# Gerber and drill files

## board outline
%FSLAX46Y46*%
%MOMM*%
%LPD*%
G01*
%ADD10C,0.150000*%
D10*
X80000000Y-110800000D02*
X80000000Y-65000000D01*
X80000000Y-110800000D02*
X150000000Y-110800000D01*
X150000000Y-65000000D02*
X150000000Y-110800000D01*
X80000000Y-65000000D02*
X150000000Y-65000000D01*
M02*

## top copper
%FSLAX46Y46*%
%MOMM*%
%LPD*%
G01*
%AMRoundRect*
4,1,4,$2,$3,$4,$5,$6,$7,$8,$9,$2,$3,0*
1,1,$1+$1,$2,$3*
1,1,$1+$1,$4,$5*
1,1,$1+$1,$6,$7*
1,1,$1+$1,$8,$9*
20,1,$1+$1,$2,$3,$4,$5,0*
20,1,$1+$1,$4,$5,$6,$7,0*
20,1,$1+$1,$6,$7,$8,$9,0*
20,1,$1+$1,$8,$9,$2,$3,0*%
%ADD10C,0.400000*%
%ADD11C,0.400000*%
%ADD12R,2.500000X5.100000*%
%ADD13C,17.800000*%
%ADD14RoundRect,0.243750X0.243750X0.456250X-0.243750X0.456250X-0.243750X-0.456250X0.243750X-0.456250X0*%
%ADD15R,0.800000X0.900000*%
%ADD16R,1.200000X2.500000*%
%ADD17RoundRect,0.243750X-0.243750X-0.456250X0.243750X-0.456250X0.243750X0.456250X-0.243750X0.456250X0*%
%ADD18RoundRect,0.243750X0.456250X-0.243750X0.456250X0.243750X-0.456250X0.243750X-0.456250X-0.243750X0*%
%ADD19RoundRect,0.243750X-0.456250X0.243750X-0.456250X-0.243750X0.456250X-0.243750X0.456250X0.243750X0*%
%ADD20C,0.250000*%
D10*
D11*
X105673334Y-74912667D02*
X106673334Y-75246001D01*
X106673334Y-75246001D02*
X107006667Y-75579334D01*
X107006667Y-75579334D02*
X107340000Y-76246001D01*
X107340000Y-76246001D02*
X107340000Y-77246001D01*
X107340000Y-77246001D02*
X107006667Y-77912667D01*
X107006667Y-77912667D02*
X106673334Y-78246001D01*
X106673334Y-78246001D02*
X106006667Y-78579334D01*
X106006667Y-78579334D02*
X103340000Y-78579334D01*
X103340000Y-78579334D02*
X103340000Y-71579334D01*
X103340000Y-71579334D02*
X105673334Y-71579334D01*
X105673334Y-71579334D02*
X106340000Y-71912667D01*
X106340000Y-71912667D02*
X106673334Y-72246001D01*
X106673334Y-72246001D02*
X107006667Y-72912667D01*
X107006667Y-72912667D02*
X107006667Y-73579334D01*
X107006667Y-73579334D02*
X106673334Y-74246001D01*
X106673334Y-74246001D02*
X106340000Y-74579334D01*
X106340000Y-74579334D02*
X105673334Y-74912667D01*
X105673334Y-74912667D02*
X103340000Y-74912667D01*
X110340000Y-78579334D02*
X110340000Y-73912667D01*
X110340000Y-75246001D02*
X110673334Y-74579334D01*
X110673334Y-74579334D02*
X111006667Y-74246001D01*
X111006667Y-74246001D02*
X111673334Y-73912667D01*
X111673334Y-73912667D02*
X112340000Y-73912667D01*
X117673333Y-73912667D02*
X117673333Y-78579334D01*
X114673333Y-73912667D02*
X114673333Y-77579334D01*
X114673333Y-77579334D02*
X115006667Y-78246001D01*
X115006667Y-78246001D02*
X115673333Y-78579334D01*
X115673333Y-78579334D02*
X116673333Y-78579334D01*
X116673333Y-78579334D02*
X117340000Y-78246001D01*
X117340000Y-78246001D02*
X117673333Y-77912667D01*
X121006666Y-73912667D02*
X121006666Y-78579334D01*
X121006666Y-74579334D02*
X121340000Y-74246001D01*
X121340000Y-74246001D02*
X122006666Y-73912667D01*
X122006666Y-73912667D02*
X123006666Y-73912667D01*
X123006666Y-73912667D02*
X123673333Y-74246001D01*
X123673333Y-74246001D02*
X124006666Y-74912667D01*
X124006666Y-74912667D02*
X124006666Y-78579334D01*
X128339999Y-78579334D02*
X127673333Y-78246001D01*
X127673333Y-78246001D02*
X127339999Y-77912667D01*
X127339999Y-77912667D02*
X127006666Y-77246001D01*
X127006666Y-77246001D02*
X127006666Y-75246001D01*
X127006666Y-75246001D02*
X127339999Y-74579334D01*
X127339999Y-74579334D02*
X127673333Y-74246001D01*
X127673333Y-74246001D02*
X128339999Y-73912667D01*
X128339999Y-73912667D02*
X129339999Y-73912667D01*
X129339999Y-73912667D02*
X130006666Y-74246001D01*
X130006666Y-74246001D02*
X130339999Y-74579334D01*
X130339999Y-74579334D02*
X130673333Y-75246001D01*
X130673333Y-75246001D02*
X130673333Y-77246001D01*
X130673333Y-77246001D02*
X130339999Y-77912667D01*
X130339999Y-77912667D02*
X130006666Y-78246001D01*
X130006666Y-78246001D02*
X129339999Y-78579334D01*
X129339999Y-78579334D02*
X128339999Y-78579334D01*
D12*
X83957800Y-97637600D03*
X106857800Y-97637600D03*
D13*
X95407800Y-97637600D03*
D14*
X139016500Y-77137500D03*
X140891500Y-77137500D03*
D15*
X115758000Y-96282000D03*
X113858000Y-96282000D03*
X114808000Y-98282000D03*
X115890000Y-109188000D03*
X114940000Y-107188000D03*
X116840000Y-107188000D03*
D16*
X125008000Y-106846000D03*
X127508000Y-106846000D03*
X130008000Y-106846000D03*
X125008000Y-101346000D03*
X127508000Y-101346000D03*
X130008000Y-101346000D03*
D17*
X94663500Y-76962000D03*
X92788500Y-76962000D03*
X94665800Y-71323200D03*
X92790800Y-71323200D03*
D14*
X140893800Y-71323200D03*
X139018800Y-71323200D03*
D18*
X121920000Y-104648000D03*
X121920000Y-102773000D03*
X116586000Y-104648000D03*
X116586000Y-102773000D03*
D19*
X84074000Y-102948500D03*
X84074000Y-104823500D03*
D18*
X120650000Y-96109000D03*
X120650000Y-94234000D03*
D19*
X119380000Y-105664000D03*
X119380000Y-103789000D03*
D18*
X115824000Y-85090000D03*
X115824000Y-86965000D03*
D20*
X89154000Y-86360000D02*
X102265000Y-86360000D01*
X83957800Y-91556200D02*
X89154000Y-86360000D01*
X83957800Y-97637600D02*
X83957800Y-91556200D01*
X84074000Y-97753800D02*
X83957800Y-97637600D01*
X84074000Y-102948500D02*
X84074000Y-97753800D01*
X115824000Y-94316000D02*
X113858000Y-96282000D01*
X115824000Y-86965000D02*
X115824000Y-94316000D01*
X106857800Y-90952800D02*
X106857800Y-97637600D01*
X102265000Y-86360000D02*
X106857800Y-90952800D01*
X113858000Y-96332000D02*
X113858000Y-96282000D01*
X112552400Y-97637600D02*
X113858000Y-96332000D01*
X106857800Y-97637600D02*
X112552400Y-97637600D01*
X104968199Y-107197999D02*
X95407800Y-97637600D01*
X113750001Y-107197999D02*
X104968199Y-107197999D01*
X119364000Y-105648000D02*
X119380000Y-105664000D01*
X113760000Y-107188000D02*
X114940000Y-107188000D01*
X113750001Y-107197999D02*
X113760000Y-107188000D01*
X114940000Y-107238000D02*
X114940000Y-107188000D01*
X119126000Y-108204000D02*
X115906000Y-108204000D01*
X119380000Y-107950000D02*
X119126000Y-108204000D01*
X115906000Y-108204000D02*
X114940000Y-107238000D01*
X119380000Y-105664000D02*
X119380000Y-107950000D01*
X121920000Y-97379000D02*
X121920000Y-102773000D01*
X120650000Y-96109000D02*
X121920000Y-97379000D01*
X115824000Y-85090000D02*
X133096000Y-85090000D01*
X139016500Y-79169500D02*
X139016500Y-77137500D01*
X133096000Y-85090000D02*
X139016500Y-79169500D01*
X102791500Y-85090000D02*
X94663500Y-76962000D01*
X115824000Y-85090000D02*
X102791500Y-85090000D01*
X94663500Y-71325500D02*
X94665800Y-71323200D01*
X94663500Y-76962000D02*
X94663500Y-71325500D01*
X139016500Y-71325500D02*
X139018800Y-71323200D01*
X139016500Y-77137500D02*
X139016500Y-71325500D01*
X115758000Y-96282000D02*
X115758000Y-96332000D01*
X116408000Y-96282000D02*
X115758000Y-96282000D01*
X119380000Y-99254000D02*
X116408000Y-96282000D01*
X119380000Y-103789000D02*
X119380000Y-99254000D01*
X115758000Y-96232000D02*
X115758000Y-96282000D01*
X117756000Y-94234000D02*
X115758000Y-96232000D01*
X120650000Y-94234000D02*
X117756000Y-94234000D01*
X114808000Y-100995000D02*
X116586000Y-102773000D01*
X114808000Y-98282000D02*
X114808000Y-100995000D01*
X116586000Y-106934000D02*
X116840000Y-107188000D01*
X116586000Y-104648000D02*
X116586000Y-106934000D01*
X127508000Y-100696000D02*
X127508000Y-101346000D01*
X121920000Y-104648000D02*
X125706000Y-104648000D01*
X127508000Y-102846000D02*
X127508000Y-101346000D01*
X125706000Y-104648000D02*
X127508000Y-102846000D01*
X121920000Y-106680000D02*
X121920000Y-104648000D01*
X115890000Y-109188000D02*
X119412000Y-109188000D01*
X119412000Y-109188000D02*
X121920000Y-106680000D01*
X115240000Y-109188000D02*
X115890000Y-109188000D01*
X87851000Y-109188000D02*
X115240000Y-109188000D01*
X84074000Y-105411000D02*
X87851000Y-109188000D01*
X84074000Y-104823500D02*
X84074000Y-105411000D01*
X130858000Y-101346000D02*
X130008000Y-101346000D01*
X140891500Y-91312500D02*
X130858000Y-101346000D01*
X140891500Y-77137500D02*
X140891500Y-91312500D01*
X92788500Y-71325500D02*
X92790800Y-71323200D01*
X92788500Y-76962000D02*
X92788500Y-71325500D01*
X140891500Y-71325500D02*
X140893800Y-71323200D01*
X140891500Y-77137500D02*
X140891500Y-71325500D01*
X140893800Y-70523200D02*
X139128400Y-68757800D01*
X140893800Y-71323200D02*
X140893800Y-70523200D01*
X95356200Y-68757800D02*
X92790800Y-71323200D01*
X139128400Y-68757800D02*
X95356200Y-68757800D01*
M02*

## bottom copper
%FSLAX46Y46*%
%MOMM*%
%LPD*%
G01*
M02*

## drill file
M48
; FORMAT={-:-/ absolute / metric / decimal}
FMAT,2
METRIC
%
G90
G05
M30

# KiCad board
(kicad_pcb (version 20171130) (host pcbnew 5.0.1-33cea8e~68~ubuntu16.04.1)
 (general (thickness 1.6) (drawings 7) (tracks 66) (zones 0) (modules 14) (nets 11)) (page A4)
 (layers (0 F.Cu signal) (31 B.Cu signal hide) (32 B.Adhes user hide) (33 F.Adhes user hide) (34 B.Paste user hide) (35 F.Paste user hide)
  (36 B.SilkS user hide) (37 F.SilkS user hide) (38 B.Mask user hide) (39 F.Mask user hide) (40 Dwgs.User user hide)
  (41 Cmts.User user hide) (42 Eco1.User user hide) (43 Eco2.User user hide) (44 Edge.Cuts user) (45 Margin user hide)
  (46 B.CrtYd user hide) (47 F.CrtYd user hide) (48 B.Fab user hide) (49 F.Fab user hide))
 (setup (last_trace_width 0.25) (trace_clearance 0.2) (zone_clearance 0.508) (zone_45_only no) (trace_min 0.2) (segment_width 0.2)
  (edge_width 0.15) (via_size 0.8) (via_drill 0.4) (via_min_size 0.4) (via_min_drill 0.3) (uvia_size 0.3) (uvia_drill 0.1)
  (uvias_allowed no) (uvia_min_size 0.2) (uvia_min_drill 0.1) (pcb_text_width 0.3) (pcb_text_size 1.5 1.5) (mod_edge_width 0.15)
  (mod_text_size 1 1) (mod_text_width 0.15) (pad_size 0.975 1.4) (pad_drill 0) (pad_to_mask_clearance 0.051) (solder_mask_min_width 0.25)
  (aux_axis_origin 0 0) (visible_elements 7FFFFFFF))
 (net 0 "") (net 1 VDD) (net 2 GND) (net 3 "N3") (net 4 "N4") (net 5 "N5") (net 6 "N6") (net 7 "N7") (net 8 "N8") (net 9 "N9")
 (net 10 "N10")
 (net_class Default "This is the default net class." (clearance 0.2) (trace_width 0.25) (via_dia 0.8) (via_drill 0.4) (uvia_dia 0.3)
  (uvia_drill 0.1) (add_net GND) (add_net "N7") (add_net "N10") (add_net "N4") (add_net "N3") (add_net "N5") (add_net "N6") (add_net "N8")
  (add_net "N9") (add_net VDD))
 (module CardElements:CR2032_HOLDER (layer F.Cu) (at 95.4078 97.6376)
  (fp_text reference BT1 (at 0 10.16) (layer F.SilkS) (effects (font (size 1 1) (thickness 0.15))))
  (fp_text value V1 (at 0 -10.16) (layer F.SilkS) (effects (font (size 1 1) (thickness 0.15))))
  (pad 1 smd rect (at -11.45 0) (size 2.5 5.1) (layers F.Cu F.Paste F.Mask) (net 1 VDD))
  (pad 1 smd rect (at 11.45 0) (size 2.5 5.1) (layers F.Cu F.Paste F.Mask) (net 1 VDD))
  (pad 2 smd circle (at 0 0) (size 17.8 17.8) (layers F.Cu F.Paste F.Mask) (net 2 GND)))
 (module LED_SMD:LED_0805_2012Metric (layer F.Cu) (at 139.954 77.1375 180)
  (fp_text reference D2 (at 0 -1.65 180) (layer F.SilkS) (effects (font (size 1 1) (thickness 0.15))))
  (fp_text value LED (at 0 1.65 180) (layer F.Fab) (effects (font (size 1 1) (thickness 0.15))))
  (pad 2 smd roundrect (at 0.9375 0 180) (size 0.975 1.4) (layers F.Cu F.Paste F.Mask) (roundrect_rratio 0.25) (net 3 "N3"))
  (pad 1 smd roundrect (at -0.9375 0 180) (size 0.975 1.4) (layers F.Cu F.Paste F.Mask) (roundrect_rratio 0.25) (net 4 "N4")))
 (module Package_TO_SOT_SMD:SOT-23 (layer F.Cu) (at 114.808 97.282 270)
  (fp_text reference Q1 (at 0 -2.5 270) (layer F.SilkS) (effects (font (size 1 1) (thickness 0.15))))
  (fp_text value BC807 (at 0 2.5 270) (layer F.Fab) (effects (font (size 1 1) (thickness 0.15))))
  (pad 1 smd rect (at -1 -0.95 270) (size 0.9 0.8) (layers F.Cu F.Paste F.Mask) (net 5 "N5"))
  (pad 2 smd rect (at -1 0.95 270) (size 0.9 0.8) (layers F.Cu F.Paste F.Mask) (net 1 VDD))
  (pad 3 smd rect (at 1 0 270) (size 0.9 0.8) (layers F.Cu F.Paste F.Mask) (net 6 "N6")))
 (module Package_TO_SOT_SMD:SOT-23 (layer F.Cu) (at 115.89 108.188 270)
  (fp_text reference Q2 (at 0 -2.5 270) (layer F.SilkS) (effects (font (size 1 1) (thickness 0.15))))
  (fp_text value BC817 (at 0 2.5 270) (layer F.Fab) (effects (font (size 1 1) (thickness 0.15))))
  (pad 3 smd rect (at 1 0 270) (size 0.9 0.8) (layers F.Cu F.Paste F.Mask) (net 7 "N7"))
  (pad 2 smd rect (at -1 0.95 270) (size 0.9 0.8) (layers F.Cu F.Paste F.Mask) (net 2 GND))
  (pad 1 smd rect (at -1 -0.95 270) (size 0.9 0.8) (layers F.Cu F.Paste F.Mask) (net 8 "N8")))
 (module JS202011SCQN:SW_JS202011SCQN (layer F.Cu) (at 127.508 104.096 180)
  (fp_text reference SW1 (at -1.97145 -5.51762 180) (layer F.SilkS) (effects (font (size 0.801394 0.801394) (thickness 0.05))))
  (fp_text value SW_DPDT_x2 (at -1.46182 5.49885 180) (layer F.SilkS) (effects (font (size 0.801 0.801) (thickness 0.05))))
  (pad 6 smd rect (at 2.5 -2.75 180) (size 1.2 2.5) (layers F.Cu F.Paste F.Mask))
  (pad 5 smd rect (at 0 -2.75 180) (size 1.2 2.5) (layers F.Cu F.Paste F.Mask))
  (pad 4 smd rect (at -2.5 -2.75 180) (size 1.2 2.5) (layers F.Cu F.Paste F.Mask))
  (pad 3 smd rect (at 2.5 2.75 180) (size 1.2 2.5) (layers F.Cu F.Paste F.Mask) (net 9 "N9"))
  (pad 2 smd rect (at 0 2.75 180) (size 1.2 2.5) (layers F.Cu F.Paste F.Mask) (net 7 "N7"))
  (pad 1 smd rect (at -2.5 2.75 180) (size 1.2 2.5) (layers F.Cu F.Paste F.Mask) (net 4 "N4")))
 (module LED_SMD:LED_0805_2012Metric (layer F.Cu) (at 93.726 76.962)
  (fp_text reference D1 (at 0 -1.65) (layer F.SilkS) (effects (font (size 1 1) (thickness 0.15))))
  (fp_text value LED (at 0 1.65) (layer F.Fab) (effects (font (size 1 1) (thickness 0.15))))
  (pad 2 smd roundrect (at 0.9375 0) (size 0.975 1.4) (layers F.Cu F.Paste F.Mask) (roundrect_rratio 0.25) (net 3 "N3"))
  (pad 1 smd roundrect (at -0.9375 0) (size 0.975 1.4) (layers F.Cu F.Paste F.Mask) (roundrect_rratio 0.25) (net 4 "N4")))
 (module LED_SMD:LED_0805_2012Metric (layer F.Cu) (at 93.7283 71.3232)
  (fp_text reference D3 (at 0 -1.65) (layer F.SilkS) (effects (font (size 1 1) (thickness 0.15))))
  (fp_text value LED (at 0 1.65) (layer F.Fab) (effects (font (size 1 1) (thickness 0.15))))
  (pad 2 smd roundrect (at 0.9375 0) (size 0.975 1.4) (layers F.Cu F.Paste F.Mask) (roundrect_rratio 0.25) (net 3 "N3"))
  (pad 1 smd roundrect (at -0.9375 0) (size 0.975 1.4) (layers F.Cu F.Paste F.Mask) (roundrect_rratio 0.25) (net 4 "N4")))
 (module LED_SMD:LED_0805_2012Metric (layer F.Cu) (at 139.9563 71.3232 180)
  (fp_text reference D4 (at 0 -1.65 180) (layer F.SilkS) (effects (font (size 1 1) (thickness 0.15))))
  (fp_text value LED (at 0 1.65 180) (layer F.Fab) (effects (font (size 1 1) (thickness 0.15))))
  (pad 1 smd roundrect (at -0.9375 0 180) (size 0.975 1.4) (layers F.Cu F.Paste F.Mask) (roundrect_rratio 0.25) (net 4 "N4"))
  (pad 2 smd roundrect (at 0.9375 0 180) (size 0.975 1.4) (layers F.Cu F.Paste F.Mask) (roundrect_rratio 0.25) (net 3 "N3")))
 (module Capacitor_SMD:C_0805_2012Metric (layer F.Cu) (at 121.92 103.7105 90)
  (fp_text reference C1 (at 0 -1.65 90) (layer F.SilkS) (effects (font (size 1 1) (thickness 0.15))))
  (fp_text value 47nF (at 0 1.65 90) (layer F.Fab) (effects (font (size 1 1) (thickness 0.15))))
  (pad 1 smd roundrect (at -0.9375 0 90) (size 0.975 1.4) (layers F.Cu F.Paste F.Mask) (roundrect_rratio 0.25) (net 7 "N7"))
  (pad 2 smd roundrect (at 0.9375 0 90) (size 0.975 1.4) (layers F.Cu F.Paste F.Mask) (roundrect_rratio 0.25) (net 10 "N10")))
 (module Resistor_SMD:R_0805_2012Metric (layer F.Cu) (at 116.586 103.7105 90)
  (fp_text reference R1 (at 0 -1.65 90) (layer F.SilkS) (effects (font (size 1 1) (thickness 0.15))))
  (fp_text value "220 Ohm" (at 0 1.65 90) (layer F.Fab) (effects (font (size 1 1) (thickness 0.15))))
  (pad 1 smd roundrect (at -0.9375 0 90) (size 0.975 1.4) (layers F.Cu F.Paste F.Mask) (roundrect_rratio 0.25) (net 8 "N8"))
  (pad 2 smd roundrect (at 0.9375 0 90) (size 0.975 1.4) (layers F.Cu F.Paste F.Mask) (roundrect_rratio 0.25) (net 6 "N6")))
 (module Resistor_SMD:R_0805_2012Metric (layer F.Cu) (at 84.074 103.886 270)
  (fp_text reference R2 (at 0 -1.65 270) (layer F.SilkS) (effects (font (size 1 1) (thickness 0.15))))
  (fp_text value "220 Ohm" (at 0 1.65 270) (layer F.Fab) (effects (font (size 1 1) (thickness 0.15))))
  (pad 1 smd roundrect (at -0.9375 0 270) (size 0.975 1.4) (layers F.Cu F.Paste F.Mask) (roundrect_rratio 0.25) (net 1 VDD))
  (pad 2 smd roundrect (at 0.9375 0 270) (size 0.975 1.4) (layers F.Cu F.Paste F.Mask) (roundrect_rratio 0.25) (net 7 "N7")))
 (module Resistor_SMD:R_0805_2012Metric (layer F.Cu) (at 120.65 95.1715 90)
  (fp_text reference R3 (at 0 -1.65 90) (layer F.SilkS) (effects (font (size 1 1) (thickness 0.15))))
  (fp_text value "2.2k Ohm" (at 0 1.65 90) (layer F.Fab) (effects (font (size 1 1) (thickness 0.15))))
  (pad 1 smd roundrect (at -0.9375 0 90) (size 0.975 1.4) (layers F.Cu F.Paste F.Mask) (roundrect_rratio 0.25) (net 10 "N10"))
  (pad 2 smd roundrect (at 0.9375 0 90) (size 0.975 1.4) (layers F.Cu F.Paste F.Mask) (roundrect_rratio 0.25) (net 5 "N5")))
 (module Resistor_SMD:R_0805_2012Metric (layer F.Cu) (at 119.38 104.7265 270)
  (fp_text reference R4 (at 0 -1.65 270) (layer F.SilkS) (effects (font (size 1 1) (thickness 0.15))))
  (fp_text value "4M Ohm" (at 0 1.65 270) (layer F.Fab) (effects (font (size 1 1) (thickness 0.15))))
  (pad 2 smd roundrect (at 0.9375 0 270) (size 0.975 1.4) (layers F.Cu F.Paste F.Mask) (roundrect_rratio 0.25) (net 2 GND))
  (pad 1 smd roundrect (at -0.9375 0 270) (size 0.975 1.4) (layers F.Cu F.Paste F.Mask) (roundrect_rratio 0.25) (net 5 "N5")))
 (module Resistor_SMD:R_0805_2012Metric (layer F.Cu) (at 115.824 86.0275 90)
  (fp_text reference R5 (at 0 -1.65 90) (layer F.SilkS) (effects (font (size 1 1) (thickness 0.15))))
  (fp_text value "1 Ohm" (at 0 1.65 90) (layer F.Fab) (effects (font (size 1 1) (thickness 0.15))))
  (pad 2 smd roundrect (at 0.9375 0 90) (size 0.975 1.4) (layers F.Cu F.Paste F.Mask) (roundrect_rratio 0.25) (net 3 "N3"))
  (pad 1 smd roundrect (at -0.9375 0 90) (size 0.975 1.4) (layers F.Cu F.Paste F.Mask) (roundrect_rratio 0.25) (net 1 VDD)))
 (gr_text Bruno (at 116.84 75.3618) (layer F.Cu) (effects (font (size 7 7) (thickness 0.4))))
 (gr_line (start 80 110.8) (end 80 65) (layer Edge.Cuts) (width 0.15))
 (gr_line (start 80 110.8) (end 150 110.8) (layer Edge.Cuts) (width 0.15))
 (gr_line (start 150 65) (end 150 110.8) (layer Edge.Cuts) (width 0.15))
 (gr_line (start 80 65) (end 150 65) (layer Edge.Cuts) (width 0.15))
 (segment (start 89.154 86.36) (end 102.265 86.36) (width 0.25) (layer F.Cu) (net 1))
 (segment (start 83.9578 91.5562) (end 89.154 86.36) (width 0.25) (layer F.Cu) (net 1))
 (segment (start 83.9578 97.6376) (end 83.9578 91.5562) (width 0.25) (layer F.Cu) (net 1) (status 10))
 (segment (start 84.074 97.7538) (end 83.9578 97.6376) (width 0.25) (layer F.Cu) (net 1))
 (segment (start 84.074 102.9485) (end 84.074 97.7538) (width 0.25) (layer F.Cu) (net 1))
 (segment (start 115.824 94.316) (end 113.858 96.282) (width 0.25) (layer F.Cu) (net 1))
 (segment (start 115.824 86.965) (end 115.824 94.316) (width 0.25) (layer F.Cu) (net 1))
 (segment (start 106.8578 90.9528) (end 106.8578 97.6376) (width 0.25) (layer F.Cu) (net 1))
 (segment (start 102.265 86.36) (end 106.8578 90.9528) (width 0.25) (layer F.Cu) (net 1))
 (segment (start 113.858 96.332) (end 113.858 96.282) (width 0.25) (layer F.Cu) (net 1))
 (segment (start 112.5524 97.6376) (end 113.858 96.332) (width 0.25) (layer F.Cu) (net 1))
 (segment (start 106.8578 97.6376) (end 112.5524 97.6376) (width 0.25) (layer F.Cu) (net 1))
 (segment (start 104.968199 107.197999) (end 95.4078 97.6376) (width 0.25) (layer F.Cu) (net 2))
 (segment (start 113.750001 107.197999) (end 104.968199 107.197999) (width 0.25) (layer F.Cu) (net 2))
 (segment (start 119.364 105.648) (end 119.38 105.664) (width 0.25) (layer F.Cu) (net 2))
 (segment (start 113.76 107.188) (end 114.94 107.188) (width 0.25) (layer F.Cu) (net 2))
 (segment (start 113.750001 107.197999) (end 113.76 107.188) (width 0.25) (layer F.Cu) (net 2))
 (segment (start 114.94 107.238) (end 114.94 107.188) (width 0.25) (layer F.Cu) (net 2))
 (segment (start 119.126 108.204) (end 115.906 108.204) (width 0.25) (layer F.Cu) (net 2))
 (segment (start 119.38 107.95) (end 119.126 108.204) (width 0.25) (layer F.Cu) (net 2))
 (segment (start 115.906 108.204) (end 114.94 107.238) (width 0.25) (layer F.Cu) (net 2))
 (segment (start 119.38 105.664) (end 119.38 107.95) (width 0.25) (layer F.Cu) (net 2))
 (segment (start 121.92 97.379) (end 121.92 102.773) (width 0.25) (layer F.Cu) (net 10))
 (segment (start 120.65 96.109) (end 121.92 97.379) (width 0.25) (layer F.Cu) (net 10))
 (segment (start 115.824 85.09) (end 133.096 85.09) (width 0.25) (layer F.Cu) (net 3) (status 10))
 (segment (start 139.0165 79.1695) (end 139.0165 77.1375) (width 0.25) (layer F.Cu) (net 3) (status 20))
 (segment (start 133.096 85.09) (end 139.0165 79.1695) (width 0.25) (layer F.Cu) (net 3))
 (segment (start 102.7915 85.09) (end 94.6635 76.962) (width 0.25) (layer F.Cu) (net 3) (status 20))
 (segment (start 115.824 85.09) (end 102.7915 85.09) (width 0.25) (layer F.Cu) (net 3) (status 10))
 (segment (start 94.6635 71.3255) (end 94.6658 71.3232) (width 0.25) (layer F.Cu) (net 3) (status 30))
 (segment (start 94.6635 76.962) (end 94.6635 71.3255) (width 0.25) (layer F.Cu) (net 3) (status 30))
 (segment (start 139.0165 71.3255) (end 139.0188 71.3232) (width 0.25) (layer F.Cu) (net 3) (status 30))
 (segment (start 139.0165 77.1375) (end 139.0165 71.3255) (width 0.25) (layer F.Cu) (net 3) (status 30))
 (segment (start 115.758 96.282) (end 115.758 96.332) (width 0.25) (layer F.Cu) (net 5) (status 30))
 (segment (start 116.408 96.282) (end 115.758 96.282) (width 0.25) (layer F.Cu) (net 5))
 (segment (start 119.38 99.254) (end 116.408 96.282) (width 0.25) (layer F.Cu) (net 5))
 (segment (start 119.38 103.789) (end 119.38 99.254) (width 0.25) (layer F.Cu) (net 5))
 (segment (start 115.758 96.232) (end 115.758 96.282) (width 0.25) (layer F.Cu) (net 5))
 (segment (start 117.756 94.234) (end 115.758 96.232) (width 0.25) (layer F.Cu) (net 5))
 (segment (start 120.65 94.234) (end 117.756 94.234) (width 0.25) (layer F.Cu) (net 5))
 (segment (start 114.808 100.995) (end 116.586 102.773) (width 0.25) (layer F.Cu) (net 6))
 (segment (start 114.808 98.282) (end 114.808 100.995) (width 0.25) (layer F.Cu) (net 6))
 (segment (start 116.586 106.934) (end 116.84 107.188) (width 0.25) (layer F.Cu) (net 8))
 (segment (start 116.586 104.648) (end 116.586 106.934) (width 0.25) (layer F.Cu) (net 8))
 (segment (start 127.508 100.696) (end 127.508 101.346) (width 0.25) (layer F.Cu) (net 7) (status 30))
 (segment (start 121.92 104.648) (end 125.706 104.648) (width 0.25) (layer F.Cu) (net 7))
 (segment (start 127.508 102.846) (end 127.508 101.346) (width 0.25) (layer F.Cu) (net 7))
 (segment (start 125.706 104.648) (end 127.508 102.846) (width 0.25) (layer F.Cu) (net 7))
 (segment (start 121.92 106.68) (end 121.92 104.648) (width 0.25) (layer F.Cu) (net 7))
 (segment (start 115.89 109.188) (end 119.412 109.188) (width 0.25) (layer F.Cu) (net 7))
 (segment (start 119.412 109.188) (end 121.92 106.68) (width 0.25) (layer F.Cu) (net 7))
 (segment (start 115.24 109.188) (end 115.89 109.188) (width 0.25) (layer F.Cu) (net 7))
 (segment (start 87.851 109.188) (end 115.24 109.188) (width 0.25) (layer F.Cu) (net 7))
 (segment (start 84.074 105.411) (end 87.851 109.188) (width 0.25) (layer F.Cu) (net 7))
 (segment (start 84.074 104.8235) (end 84.074 105.411) (width 0.25) (layer F.Cu) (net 7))
 (segment (start 130.858 101.346) (end 130.008 101.346) (width 0.25) (layer F.Cu) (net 4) (status 20))
 (segment (start 140.8915 91.3125) (end 130.858 101.346) (width 0.25) (layer F.Cu) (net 4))
 (segment (start 140.8915 77.1375) (end 140.8915 91.3125) (width 0.25) (layer F.Cu) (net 4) (status 10))
 (segment (start 92.7885 71.3255) (end 92.7908 71.3232) (width 0.25) (layer F.Cu) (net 4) (status 30))
 (segment (start 92.7885 76.962) (end 92.7885 71.3255) (width 0.25) (layer F.Cu) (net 4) (status 30))
 (segment (start 140.8915 71.3255) (end 140.8938 71.3232) (width 0.25) (layer F.Cu) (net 4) (status 30))
 (segment (start 140.8915 77.1375) (end 140.8915 71.3255) (width 0.25) (layer F.Cu) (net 4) (status 30))
 (segment (start 140.8938 70.5232) (end 139.1284 68.7578) (width 0.25) (layer F.Cu) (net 4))
 (segment (start 140.8938 71.3232) (end 140.8938 70.5232) (width 0.25) (layer F.Cu) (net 4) (status 10))
 (segment (start 95.3562 68.7578) (end 92.7908 71.3232) (width 0.25) (layer F.Cu) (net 4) (status 20))
 (segment (start 139.1284 68.7578) (end 95.3562 68.7578) (width 0.25) (layer F.Cu) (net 4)))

